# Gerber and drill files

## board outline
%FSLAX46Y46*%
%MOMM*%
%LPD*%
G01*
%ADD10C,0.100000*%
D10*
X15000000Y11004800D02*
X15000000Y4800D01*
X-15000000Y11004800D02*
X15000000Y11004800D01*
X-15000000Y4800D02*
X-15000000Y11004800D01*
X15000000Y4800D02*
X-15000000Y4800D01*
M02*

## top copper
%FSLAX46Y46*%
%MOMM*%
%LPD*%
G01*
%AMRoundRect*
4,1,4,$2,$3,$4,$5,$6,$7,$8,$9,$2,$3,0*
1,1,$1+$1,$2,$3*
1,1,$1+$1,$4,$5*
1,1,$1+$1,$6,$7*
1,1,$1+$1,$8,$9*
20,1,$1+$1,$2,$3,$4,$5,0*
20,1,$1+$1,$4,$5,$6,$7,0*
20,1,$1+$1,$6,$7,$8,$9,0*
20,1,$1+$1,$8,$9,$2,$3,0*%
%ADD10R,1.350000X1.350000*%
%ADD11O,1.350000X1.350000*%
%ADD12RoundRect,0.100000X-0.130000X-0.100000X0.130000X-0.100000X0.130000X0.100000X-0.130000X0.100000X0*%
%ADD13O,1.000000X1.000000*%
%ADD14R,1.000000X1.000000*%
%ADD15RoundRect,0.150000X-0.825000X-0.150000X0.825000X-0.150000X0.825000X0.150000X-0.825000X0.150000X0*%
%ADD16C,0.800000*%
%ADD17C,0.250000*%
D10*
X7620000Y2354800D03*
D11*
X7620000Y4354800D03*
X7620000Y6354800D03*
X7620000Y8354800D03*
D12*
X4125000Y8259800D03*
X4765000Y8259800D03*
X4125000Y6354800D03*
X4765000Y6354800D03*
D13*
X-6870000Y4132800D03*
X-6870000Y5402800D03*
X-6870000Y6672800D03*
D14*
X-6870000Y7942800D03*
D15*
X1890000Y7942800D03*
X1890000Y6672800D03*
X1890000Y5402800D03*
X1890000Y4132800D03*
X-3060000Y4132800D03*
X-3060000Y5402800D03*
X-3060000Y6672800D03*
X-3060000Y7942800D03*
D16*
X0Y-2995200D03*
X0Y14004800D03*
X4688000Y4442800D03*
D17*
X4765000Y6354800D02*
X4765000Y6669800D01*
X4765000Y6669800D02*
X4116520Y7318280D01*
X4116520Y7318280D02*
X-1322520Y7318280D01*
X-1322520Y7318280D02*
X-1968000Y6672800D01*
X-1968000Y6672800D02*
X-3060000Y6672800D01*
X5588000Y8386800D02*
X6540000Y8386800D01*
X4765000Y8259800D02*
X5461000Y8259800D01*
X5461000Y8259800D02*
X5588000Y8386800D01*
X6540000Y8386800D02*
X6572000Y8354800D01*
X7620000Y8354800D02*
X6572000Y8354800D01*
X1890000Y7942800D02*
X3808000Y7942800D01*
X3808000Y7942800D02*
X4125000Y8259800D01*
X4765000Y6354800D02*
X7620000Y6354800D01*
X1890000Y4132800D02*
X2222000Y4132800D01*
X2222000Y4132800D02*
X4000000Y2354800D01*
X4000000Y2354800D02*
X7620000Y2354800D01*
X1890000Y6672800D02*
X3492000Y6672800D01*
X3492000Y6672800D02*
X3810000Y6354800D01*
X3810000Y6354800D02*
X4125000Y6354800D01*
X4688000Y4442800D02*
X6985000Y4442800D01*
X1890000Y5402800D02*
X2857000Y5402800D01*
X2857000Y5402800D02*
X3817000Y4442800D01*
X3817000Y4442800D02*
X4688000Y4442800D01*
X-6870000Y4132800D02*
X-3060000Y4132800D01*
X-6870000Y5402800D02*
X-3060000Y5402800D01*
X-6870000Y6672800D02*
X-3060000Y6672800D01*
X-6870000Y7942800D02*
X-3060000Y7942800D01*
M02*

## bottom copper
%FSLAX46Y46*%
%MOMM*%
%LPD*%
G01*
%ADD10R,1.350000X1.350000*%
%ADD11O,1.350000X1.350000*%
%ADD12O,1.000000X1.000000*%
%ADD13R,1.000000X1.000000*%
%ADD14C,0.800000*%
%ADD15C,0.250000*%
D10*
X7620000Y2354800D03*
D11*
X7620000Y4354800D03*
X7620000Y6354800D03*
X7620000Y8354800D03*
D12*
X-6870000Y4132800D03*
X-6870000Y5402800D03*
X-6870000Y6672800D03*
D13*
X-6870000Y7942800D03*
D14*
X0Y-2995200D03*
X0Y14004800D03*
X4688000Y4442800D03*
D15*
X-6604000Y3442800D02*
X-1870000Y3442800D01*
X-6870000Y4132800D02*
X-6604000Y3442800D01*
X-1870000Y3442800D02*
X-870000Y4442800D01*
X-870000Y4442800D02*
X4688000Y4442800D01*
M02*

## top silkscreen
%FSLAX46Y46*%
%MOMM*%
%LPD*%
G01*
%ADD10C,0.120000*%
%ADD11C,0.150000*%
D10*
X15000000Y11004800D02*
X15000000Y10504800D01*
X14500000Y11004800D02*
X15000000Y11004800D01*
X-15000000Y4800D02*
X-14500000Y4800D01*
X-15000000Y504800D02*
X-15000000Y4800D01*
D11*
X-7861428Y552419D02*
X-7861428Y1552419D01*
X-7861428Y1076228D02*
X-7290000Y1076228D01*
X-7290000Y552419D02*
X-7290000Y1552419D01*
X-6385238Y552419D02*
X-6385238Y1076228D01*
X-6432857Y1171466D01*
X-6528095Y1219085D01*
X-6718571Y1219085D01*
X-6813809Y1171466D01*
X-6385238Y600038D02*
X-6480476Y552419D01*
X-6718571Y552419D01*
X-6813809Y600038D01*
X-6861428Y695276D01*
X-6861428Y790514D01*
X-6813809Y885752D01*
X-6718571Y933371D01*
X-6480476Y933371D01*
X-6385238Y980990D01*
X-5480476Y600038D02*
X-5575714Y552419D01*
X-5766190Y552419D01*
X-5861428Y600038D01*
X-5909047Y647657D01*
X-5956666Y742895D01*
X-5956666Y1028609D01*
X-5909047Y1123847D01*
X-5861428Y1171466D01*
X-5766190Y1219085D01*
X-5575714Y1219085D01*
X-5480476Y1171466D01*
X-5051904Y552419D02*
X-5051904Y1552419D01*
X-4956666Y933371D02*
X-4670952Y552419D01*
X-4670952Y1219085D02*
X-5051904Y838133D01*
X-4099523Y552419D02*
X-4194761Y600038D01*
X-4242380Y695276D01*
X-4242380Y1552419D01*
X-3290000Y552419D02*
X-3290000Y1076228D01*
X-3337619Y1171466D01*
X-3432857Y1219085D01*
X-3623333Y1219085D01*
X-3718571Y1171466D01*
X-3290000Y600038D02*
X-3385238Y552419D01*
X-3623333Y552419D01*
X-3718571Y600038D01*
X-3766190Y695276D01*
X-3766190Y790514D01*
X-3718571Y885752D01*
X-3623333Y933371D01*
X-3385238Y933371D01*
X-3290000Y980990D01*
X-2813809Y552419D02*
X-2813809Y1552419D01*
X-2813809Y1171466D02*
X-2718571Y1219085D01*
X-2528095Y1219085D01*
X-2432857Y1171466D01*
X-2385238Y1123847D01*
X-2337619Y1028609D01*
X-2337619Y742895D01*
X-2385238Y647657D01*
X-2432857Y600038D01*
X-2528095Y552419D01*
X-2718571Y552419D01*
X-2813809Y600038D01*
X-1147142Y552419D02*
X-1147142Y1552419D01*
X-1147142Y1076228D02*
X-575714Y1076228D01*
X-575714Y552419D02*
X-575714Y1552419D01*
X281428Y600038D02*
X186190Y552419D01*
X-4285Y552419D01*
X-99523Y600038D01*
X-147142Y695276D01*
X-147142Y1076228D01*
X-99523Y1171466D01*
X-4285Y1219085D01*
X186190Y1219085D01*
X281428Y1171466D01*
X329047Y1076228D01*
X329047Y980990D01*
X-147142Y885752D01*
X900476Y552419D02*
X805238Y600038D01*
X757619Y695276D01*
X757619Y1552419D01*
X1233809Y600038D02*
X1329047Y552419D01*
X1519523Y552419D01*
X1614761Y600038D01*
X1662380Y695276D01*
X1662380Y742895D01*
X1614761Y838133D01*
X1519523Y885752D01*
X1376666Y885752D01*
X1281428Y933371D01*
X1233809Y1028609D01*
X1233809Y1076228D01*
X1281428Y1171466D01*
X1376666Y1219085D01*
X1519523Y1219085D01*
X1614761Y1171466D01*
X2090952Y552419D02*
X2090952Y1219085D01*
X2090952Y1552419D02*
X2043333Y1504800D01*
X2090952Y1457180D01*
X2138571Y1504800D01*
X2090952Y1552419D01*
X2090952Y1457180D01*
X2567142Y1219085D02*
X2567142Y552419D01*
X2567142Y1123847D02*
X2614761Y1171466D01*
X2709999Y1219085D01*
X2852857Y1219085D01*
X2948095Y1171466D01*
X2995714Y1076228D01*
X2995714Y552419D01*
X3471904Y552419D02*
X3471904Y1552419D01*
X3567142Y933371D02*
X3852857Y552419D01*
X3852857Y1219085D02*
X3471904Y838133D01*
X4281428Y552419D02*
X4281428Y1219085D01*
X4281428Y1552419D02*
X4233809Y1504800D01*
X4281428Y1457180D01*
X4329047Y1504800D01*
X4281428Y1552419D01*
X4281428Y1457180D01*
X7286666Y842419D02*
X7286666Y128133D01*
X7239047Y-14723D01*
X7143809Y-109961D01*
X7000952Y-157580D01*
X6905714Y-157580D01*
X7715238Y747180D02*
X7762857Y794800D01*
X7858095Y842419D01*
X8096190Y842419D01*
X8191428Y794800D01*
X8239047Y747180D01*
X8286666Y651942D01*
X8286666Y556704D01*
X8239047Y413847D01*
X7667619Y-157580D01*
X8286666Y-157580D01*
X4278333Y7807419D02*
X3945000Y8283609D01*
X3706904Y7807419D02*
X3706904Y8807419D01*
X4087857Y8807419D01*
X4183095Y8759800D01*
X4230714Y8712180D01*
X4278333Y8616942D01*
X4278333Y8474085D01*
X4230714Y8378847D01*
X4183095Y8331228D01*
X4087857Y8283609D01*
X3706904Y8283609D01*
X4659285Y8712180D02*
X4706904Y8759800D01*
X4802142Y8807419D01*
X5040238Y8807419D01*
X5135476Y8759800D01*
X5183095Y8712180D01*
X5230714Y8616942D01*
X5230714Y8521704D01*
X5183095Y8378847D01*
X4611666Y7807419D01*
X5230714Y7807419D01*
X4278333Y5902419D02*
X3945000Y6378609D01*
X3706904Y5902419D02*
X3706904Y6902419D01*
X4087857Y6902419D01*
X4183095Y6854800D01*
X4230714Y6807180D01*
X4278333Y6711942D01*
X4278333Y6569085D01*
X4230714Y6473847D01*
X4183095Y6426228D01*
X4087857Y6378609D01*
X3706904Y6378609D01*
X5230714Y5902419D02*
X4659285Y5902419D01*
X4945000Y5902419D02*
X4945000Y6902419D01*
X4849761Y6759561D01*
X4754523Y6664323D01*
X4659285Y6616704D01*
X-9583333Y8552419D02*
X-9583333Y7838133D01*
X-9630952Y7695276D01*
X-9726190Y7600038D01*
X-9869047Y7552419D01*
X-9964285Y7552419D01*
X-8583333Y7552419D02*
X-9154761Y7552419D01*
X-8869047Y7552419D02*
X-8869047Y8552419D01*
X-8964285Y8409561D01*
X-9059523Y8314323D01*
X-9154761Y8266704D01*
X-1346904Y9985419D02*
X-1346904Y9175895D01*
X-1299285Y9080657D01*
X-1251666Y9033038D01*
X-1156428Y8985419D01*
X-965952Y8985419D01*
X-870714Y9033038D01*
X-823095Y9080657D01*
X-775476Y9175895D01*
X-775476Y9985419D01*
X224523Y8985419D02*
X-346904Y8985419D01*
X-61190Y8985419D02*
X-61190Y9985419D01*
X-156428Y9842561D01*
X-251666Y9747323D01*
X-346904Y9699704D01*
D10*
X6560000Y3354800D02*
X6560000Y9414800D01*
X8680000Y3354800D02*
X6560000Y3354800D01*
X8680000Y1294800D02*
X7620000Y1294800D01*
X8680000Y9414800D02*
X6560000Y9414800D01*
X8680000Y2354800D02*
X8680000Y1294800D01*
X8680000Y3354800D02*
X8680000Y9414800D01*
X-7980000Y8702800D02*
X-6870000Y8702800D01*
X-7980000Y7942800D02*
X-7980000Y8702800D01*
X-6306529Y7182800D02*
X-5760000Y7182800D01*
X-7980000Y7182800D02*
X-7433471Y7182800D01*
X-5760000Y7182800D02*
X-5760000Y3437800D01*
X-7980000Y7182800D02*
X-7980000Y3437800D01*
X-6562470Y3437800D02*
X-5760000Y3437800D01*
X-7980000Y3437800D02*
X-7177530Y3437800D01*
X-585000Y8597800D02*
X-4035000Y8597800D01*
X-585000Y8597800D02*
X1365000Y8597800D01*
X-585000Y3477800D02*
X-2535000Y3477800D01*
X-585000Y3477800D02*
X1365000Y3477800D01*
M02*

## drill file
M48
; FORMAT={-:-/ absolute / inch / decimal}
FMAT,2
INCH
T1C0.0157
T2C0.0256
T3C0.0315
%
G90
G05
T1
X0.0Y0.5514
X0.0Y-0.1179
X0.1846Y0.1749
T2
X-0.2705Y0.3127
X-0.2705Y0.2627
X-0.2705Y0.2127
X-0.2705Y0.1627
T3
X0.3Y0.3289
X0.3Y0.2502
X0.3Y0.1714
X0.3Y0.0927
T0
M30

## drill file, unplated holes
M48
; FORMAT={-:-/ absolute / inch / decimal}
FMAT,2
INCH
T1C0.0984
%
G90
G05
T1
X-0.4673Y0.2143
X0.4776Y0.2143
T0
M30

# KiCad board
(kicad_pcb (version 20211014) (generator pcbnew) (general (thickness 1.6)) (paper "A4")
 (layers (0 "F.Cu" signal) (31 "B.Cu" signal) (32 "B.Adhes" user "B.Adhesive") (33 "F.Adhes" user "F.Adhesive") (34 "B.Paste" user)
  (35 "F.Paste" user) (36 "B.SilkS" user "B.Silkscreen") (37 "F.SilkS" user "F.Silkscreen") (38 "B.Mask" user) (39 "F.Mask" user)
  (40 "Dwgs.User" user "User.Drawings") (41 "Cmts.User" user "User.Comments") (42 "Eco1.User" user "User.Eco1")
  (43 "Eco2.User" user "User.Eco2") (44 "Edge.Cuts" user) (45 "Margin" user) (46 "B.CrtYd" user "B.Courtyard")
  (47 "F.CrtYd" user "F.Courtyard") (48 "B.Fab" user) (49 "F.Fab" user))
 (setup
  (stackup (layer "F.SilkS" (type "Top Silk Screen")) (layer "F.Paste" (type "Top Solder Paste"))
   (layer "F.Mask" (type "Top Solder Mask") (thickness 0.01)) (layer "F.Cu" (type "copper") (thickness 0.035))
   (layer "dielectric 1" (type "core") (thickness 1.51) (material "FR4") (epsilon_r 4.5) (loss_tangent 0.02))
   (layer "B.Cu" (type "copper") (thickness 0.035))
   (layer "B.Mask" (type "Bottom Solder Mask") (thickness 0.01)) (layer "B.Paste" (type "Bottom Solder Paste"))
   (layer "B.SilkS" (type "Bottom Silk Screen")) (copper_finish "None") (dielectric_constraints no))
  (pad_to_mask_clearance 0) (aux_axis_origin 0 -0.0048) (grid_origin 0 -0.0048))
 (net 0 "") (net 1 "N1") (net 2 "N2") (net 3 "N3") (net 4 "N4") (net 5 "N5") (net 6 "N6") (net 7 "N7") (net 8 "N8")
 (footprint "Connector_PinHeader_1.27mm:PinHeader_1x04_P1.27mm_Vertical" (layer "F.Cu") (at -6.87 -7.9428)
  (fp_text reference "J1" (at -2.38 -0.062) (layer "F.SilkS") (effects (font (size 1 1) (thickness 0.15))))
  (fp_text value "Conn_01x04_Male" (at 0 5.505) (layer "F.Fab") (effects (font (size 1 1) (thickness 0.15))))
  (fp_line (start -1.11 -0.76) (end 0 -0.76) (layer "F.SilkS") (width 0.12))
  (fp_line (start 0.30753 4.505) (end 1.11 4.505) (layer "F.SilkS") (width 0.12))
  (fp_line (start -1.11 0) (end -1.11 -0.76) (layer "F.SilkS") (width 0.12))
  (fp_line (start 1.11 0.76) (end 1.11 4.505) (layer "F.SilkS") (width 0.12))
  (fp_line (start 0.563471 0.76) (end 1.11 0.76) (layer "F.SilkS") (width 0.12))
  (fp_line (start -1.11 0.76) (end -0.563471 0.76) (layer "F.SilkS") (width 0.12))
  (fp_line (start -1.11 0.76) (end -1.11 4.505) (layer "F.SilkS") (width 0.12))
  (fp_line (start -1.11 4.505) (end -0.30753 4.505) (layer "F.SilkS") (width 0.12))
  (pad "1" thru_hole rect locked (at 0 0) (size 1 1) (drill 0.65) (layers *.Cu *.Mask) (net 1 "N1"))
  (pad "2" thru_hole oval locked (at 0 1.27) (size 1 1) (drill 0.65) (layers *.Cu *.Mask) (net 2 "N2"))
  (pad "3" thru_hole oval locked (at 0 2.54) (size 1 1) (drill 0.65) (layers *.Cu *.Mask) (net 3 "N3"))
  (pad "4" thru_hole oval locked (at 0 3.81) (size 1 1) (drill 0.65) (layers *.Cu *.Mask) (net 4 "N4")))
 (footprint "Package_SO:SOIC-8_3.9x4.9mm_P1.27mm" (layer "F.Cu") (at -0.585 -6.0378)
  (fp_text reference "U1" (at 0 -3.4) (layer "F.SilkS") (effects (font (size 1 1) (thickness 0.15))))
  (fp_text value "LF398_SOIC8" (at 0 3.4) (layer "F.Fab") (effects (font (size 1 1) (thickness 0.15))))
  (fp_line (start 0 -2.56) (end -3.45 -2.56) (layer "F.SilkS") (width 0.12))
  (fp_line (start 0 2.56) (end -1.95 2.56) (layer "F.SilkS") (width 0.12))
  (fp_line (start 0 2.56) (end 1.95 2.56) (layer "F.SilkS") (width 0.12))
  (fp_line (start 0 -2.56) (end 1.95 -2.56) (layer "F.SilkS") (width 0.12))
  (pad "1" smd roundrect locked (at -2.475 -1.905) (size 1.95 0.6) (layers "F.Cu" "F.Paste" "F.Mask") (roundrect_rratio 0.25) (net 1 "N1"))
  (pad "2" smd roundrect locked (at -2.475 -0.635) (size 1.95 0.6) (layers "F.Cu" "F.Paste" "F.Mask") (roundrect_rratio 0.25) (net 2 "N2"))
  (pad "3" smd roundrect locked (at -2.475 0.635) (size 1.95 0.6) (layers "F.Cu" "F.Paste" "F.Mask") (roundrect_rratio 0.25) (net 3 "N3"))
  (pad "4" smd roundrect locked (at -2.475 1.905) (size 1.95 0.6) (layers "F.Cu" "F.Paste" "F.Mask") (roundrect_rratio 0.25) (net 4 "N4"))
  (pad "5" smd roundrect locked (at 2.475 1.905) (size 1.95 0.6) (layers "F.Cu" "F.Paste" "F.Mask") (roundrect_rratio 0.25) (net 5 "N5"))
  (pad "6" smd roundrect locked (at 2.475 0.635) (size 1.95 0.6) (layers "F.Cu" "F.Paste" "F.Mask") (roundrect_rratio 0.25) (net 4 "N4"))
  (pad "7" smd roundrect locked (at 2.475 -0.635) (size 1.95 0.6) (layers "F.Cu" "F.Paste" "F.Mask") (roundrect_rratio 0.25) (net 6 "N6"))
  (pad "8" smd roundrect locked (at 2.475 -1.905) (size 1.95 0.6) (layers "F.Cu" "F.Paste" "F.Mask") (roundrect_rratio 0.25) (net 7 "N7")))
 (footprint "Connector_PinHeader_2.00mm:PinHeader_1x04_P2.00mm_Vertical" (layer "F.Cu") (at 7.62 -2.3548 180)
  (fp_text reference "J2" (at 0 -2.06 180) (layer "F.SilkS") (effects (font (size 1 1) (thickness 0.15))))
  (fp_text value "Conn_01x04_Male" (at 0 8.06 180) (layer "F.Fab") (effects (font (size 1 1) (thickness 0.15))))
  (fp_line (start -1.06 1) (end -1.06 7.06) (layer "F.SilkS") (width 0.12))
  (fp_line (start -1.06 1) (end 1.06 1) (layer "F.SilkS") (width 0.12))
  (fp_line (start -1.06 0) (end -1.06 -1.06) (layer "F.SilkS") (width 0.12))
  (fp_line (start -1.06 -1.06) (end 0 -1.06) (layer "F.SilkS") (width 0.12))
  (fp_line (start -1.06 7.06) (end 1.06 7.06) (layer "F.SilkS") (width 0.12))
  (fp_line (start 1.06 1) (end 1.06 7.06) (layer "F.SilkS") (width 0.12))
  (pad "1" thru_hole rect (at 0 0 180) (size 1.35 1.35) (drill 0.8) (layers *.Cu *.Mask) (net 5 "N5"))
  (pad "2" thru_hole oval (at 0 2 180) (size 1.35 1.35) (drill 0.8) (layers *.Cu *.Mask) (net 4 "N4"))
  (pad "3" thru_hole oval (at 0 4 180) (size 1.35 1.35) (drill 0.8) (layers *.Cu *.Mask) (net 2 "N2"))
  (pad "4" thru_hole oval (at 0 6 180) (size 1.35 1.35) (drill 0.8) (layers *.Cu *.Mask) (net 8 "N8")))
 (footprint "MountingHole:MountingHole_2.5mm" (layer "F.Cu") (at -11.87 -5.4428)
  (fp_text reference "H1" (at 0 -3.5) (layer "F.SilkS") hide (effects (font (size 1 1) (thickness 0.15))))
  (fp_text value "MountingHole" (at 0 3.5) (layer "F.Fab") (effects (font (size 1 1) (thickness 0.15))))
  (pad "" np_thru_hole circle locked (at 0 0) (size 2.5 2.5) (drill 2.5) (layers *.Cu *.Mask)))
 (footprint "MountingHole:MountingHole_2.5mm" (layer "F.Cu") (at 12.13 -5.4428)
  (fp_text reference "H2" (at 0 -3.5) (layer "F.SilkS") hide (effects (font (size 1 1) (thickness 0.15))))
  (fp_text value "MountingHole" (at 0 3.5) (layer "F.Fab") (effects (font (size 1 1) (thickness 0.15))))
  (pad "" np_thru_hole circle locked (at 0 0) (size 2.5 2.5) (drill 2.5) (layers *.Cu *.Mask)))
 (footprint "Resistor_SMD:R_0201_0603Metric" (layer "F.Cu") (at 4.445 -6.3548)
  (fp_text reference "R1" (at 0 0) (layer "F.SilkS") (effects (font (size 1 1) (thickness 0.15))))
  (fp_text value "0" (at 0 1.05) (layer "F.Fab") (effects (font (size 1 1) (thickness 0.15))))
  (pad "" smd roundrect (at -0.345 0) (size 0.318 0.36) (layers "F.Paste") (roundrect_rratio 0.25))
  (pad "" smd roundrect (at 0.345 0) (size 0.318 0.36) (layers "F.Paste") (roundrect_rratio 0.25))
  (pad "1" smd roundrect (at -0.32 0) (size 0.46 0.4) (layers "F.Cu" "F.Mask") (roundrect_rratio 0.25) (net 6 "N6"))
  (pad "2" smd roundrect (at 0.32 0) (size 0.46 0.4) (layers "F.Cu" "F.Mask") (roundrect_rratio 0.25) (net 2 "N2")))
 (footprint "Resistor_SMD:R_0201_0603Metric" (layer "F.Cu") (at 4.445 -8.2598)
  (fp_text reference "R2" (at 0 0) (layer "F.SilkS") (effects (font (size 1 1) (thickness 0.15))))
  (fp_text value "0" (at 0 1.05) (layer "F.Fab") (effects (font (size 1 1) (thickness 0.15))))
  (pad "" smd roundrect (at -0.345 0) (size 0.318 0.36) (layers "F.Paste") (roundrect_rratio 0.25))
  (pad "" smd roundrect (at 0.345 0) (size 0.318 0.36) (layers "F.Paste") (roundrect_rratio 0.25))
  (pad "1" smd roundrect (at -0.32 0) (size 0.46 0.4) (layers "F.Cu" "F.Mask") (roundrect_rratio 0.25) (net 7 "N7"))
  (pad "2" smd roundrect (at 0.32 0) (size 0.46 0.4) (layers "F.Cu" "F.Mask") (roundrect_rratio 0.25) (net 8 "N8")))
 (gr_line (start 15 -11.0048) (end 15 -10.5048) (layer "F.SilkS") (width 0.12))
 (gr_line (start -15 -0.0048) (end -14.5 -0.0048) (layer "F.SilkS") (width 0.12))
 (gr_line (start 14.5 -11.0048) (end 15 -11.0048) (layer "F.SilkS") (width 0.12))
 (gr_line (start -15 -0.5048) (end -15 -0.0048) (layer "F.SilkS") (width 0.12))
 (gr_line (start -15 -11.0048) (end 15 -11.0048) (layer "Edge.Cuts") (width 0.1))
 (gr_line (start 15 -11.0048) (end 15 -0.0048) (layer "Edge.Cuts") (width 0.1))
 (gr_line (start 15 -0.0048) (end -15 -0.0048) (layer "Edge.Cuts") (width 0.1))
 (gr_line (start -15 -0.0048) (end -15 -11.0048) (layer "Edge.Cuts") (width 0.1))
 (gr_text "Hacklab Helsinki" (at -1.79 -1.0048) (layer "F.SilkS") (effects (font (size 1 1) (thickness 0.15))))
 (via (at 0 2.9952) (size 0.8) (drill 0.4) (layers "F.Cu" "B.Cu") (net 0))
 (via (at 0 -14.0048) (size 0.8) (drill 0.4) (layers "F.Cu" "B.Cu") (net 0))
 (segment (start 1.89 -5.4028) (end 2.857 -5.4028) (width 0.25) (layer "F.Cu") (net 4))
 (segment (start 3.817 -4.4428) (end 4.688 -4.4428) (width 0.25) (layer "F.Cu") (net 4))
 (segment (start -6.87 -4.1328) (end -3.06 -4.1328) (width 0.25) (layer "F.Cu") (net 4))
 (segment (start 2.857 -5.4028) (end 3.817 -4.4428) (width 0.25) (layer "F.Cu") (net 4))
 (segment (start 4.688 -4.4428) (end 6.985 -4.4428) (width 0.25) (layer "F.Cu") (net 4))
 (via (at 4.688 -4.4428) (size 0.8) (drill 0.4) (layers "F.Cu" "B.Cu") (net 4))
 (segment (start -6.87 -4.1328) (end -6.604 -3.4428) (width 0.25) (layer "B.Cu") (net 4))
 (segment (start -0.87 -4.4428) (end 4.688 -4.4428) (width 0.25) (layer "B.Cu") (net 4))
 (segment (start -1.87 -3.4428) (end -0.87 -4.4428) (width 0.25) (layer "B.Cu") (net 4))
 (segment (start -6.604 -3.4428) (end -1.87 -3.4428) (width 0.25) (layer "B.Cu") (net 4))
 (segment (start -6.87 -5.4028) (end -3.06 -5.4028) (width 0.25) (layer "F.Cu") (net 3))
 (segment (start -6.87 -6.6728) (end -3.06 -6.6728) (width 0.25) (layer "F.Cu") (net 2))
 (segment (start 4.11652 -7.31828) (end -1.32252 -7.31828) (width 0.25) (layer "F.Cu") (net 2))
 (segment (start 4.765 -6.3548) (end 4.765 -6.6698) (width 0.25) (layer "F.Cu") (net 2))
 (segment (start -1.968 -6.6728) (end -3.06 -6.6728) (width 0.25) (layer "F.Cu") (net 2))
 (segment (start 4.765 -6.3548) (end 7.62 -6.3548) (width 0.25) (layer "F.Cu") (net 2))
 (segment (start 4.765 -6.6698) (end 4.11652 -7.31828) (width 0.25) (layer "F.Cu") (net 2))
 (segment (start -1.32252 -7.31828) (end -1.968 -6.6728) (width 0.25) (layer "F.Cu") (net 2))
 (segment (start -6.87 -7.9428) (end -3.06 -7.9428) (width 0.25) (layer "F.Cu") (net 1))
 (segment (start 6.54 -8.3868) (end 6.572 -8.3548) (width 0.25) (layer "F.Cu") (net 8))
 (segment (start 5.588 -8.3868) (end 6.54 -8.3868) (width 0.25) (layer "F.Cu") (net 8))
 (segment (start 5.461 -8.2598) (end 5.588 -8.3868) (width 0.25) (layer "F.Cu") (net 8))
 (segment (start 7.62 -8.3548) (end 6.572 -8.3548) (width 0.25) (layer "F.Cu") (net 8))
 (segment (start 4.765 -8.2598) (end 5.461 -8.2598) (width 0.25) (layer "F.Cu") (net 8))
 (segment (start 4 -2.3548) (end 7.62 -2.3548) (width 0.25) (layer "F.Cu") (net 5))
 (segment (start 2.222 -4.1328) (end 4 -2.3548) (width 0.25) (layer "F.Cu") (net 5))
 (segment (start 1.89 -4.1328) (end 2.222 -4.1328) (width 0.25) (layer "F.Cu") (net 5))
 (segment (start 3.81 -6.3548) (end 4.125 -6.3548) (width 0.25) (layer "F.Cu") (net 6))
 (segment (start 1.89 -6.6728) (end 3.492 -6.6728) (width 0.25) (layer "F.Cu") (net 6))
 (segment (start 3.492 -6.6728) (end 3.81 -6.3548) (width 0.25) (layer "F.Cu") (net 6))
 (segment (start 1.89 -7.9428) (end 3.808 -7.9428) (width 0.25) (layer "F.Cu") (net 7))
 (segment (start 3.808 -7.9428) (end 4.125 -8.2598) (width 0.25) (layer "F.Cu") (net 7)))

